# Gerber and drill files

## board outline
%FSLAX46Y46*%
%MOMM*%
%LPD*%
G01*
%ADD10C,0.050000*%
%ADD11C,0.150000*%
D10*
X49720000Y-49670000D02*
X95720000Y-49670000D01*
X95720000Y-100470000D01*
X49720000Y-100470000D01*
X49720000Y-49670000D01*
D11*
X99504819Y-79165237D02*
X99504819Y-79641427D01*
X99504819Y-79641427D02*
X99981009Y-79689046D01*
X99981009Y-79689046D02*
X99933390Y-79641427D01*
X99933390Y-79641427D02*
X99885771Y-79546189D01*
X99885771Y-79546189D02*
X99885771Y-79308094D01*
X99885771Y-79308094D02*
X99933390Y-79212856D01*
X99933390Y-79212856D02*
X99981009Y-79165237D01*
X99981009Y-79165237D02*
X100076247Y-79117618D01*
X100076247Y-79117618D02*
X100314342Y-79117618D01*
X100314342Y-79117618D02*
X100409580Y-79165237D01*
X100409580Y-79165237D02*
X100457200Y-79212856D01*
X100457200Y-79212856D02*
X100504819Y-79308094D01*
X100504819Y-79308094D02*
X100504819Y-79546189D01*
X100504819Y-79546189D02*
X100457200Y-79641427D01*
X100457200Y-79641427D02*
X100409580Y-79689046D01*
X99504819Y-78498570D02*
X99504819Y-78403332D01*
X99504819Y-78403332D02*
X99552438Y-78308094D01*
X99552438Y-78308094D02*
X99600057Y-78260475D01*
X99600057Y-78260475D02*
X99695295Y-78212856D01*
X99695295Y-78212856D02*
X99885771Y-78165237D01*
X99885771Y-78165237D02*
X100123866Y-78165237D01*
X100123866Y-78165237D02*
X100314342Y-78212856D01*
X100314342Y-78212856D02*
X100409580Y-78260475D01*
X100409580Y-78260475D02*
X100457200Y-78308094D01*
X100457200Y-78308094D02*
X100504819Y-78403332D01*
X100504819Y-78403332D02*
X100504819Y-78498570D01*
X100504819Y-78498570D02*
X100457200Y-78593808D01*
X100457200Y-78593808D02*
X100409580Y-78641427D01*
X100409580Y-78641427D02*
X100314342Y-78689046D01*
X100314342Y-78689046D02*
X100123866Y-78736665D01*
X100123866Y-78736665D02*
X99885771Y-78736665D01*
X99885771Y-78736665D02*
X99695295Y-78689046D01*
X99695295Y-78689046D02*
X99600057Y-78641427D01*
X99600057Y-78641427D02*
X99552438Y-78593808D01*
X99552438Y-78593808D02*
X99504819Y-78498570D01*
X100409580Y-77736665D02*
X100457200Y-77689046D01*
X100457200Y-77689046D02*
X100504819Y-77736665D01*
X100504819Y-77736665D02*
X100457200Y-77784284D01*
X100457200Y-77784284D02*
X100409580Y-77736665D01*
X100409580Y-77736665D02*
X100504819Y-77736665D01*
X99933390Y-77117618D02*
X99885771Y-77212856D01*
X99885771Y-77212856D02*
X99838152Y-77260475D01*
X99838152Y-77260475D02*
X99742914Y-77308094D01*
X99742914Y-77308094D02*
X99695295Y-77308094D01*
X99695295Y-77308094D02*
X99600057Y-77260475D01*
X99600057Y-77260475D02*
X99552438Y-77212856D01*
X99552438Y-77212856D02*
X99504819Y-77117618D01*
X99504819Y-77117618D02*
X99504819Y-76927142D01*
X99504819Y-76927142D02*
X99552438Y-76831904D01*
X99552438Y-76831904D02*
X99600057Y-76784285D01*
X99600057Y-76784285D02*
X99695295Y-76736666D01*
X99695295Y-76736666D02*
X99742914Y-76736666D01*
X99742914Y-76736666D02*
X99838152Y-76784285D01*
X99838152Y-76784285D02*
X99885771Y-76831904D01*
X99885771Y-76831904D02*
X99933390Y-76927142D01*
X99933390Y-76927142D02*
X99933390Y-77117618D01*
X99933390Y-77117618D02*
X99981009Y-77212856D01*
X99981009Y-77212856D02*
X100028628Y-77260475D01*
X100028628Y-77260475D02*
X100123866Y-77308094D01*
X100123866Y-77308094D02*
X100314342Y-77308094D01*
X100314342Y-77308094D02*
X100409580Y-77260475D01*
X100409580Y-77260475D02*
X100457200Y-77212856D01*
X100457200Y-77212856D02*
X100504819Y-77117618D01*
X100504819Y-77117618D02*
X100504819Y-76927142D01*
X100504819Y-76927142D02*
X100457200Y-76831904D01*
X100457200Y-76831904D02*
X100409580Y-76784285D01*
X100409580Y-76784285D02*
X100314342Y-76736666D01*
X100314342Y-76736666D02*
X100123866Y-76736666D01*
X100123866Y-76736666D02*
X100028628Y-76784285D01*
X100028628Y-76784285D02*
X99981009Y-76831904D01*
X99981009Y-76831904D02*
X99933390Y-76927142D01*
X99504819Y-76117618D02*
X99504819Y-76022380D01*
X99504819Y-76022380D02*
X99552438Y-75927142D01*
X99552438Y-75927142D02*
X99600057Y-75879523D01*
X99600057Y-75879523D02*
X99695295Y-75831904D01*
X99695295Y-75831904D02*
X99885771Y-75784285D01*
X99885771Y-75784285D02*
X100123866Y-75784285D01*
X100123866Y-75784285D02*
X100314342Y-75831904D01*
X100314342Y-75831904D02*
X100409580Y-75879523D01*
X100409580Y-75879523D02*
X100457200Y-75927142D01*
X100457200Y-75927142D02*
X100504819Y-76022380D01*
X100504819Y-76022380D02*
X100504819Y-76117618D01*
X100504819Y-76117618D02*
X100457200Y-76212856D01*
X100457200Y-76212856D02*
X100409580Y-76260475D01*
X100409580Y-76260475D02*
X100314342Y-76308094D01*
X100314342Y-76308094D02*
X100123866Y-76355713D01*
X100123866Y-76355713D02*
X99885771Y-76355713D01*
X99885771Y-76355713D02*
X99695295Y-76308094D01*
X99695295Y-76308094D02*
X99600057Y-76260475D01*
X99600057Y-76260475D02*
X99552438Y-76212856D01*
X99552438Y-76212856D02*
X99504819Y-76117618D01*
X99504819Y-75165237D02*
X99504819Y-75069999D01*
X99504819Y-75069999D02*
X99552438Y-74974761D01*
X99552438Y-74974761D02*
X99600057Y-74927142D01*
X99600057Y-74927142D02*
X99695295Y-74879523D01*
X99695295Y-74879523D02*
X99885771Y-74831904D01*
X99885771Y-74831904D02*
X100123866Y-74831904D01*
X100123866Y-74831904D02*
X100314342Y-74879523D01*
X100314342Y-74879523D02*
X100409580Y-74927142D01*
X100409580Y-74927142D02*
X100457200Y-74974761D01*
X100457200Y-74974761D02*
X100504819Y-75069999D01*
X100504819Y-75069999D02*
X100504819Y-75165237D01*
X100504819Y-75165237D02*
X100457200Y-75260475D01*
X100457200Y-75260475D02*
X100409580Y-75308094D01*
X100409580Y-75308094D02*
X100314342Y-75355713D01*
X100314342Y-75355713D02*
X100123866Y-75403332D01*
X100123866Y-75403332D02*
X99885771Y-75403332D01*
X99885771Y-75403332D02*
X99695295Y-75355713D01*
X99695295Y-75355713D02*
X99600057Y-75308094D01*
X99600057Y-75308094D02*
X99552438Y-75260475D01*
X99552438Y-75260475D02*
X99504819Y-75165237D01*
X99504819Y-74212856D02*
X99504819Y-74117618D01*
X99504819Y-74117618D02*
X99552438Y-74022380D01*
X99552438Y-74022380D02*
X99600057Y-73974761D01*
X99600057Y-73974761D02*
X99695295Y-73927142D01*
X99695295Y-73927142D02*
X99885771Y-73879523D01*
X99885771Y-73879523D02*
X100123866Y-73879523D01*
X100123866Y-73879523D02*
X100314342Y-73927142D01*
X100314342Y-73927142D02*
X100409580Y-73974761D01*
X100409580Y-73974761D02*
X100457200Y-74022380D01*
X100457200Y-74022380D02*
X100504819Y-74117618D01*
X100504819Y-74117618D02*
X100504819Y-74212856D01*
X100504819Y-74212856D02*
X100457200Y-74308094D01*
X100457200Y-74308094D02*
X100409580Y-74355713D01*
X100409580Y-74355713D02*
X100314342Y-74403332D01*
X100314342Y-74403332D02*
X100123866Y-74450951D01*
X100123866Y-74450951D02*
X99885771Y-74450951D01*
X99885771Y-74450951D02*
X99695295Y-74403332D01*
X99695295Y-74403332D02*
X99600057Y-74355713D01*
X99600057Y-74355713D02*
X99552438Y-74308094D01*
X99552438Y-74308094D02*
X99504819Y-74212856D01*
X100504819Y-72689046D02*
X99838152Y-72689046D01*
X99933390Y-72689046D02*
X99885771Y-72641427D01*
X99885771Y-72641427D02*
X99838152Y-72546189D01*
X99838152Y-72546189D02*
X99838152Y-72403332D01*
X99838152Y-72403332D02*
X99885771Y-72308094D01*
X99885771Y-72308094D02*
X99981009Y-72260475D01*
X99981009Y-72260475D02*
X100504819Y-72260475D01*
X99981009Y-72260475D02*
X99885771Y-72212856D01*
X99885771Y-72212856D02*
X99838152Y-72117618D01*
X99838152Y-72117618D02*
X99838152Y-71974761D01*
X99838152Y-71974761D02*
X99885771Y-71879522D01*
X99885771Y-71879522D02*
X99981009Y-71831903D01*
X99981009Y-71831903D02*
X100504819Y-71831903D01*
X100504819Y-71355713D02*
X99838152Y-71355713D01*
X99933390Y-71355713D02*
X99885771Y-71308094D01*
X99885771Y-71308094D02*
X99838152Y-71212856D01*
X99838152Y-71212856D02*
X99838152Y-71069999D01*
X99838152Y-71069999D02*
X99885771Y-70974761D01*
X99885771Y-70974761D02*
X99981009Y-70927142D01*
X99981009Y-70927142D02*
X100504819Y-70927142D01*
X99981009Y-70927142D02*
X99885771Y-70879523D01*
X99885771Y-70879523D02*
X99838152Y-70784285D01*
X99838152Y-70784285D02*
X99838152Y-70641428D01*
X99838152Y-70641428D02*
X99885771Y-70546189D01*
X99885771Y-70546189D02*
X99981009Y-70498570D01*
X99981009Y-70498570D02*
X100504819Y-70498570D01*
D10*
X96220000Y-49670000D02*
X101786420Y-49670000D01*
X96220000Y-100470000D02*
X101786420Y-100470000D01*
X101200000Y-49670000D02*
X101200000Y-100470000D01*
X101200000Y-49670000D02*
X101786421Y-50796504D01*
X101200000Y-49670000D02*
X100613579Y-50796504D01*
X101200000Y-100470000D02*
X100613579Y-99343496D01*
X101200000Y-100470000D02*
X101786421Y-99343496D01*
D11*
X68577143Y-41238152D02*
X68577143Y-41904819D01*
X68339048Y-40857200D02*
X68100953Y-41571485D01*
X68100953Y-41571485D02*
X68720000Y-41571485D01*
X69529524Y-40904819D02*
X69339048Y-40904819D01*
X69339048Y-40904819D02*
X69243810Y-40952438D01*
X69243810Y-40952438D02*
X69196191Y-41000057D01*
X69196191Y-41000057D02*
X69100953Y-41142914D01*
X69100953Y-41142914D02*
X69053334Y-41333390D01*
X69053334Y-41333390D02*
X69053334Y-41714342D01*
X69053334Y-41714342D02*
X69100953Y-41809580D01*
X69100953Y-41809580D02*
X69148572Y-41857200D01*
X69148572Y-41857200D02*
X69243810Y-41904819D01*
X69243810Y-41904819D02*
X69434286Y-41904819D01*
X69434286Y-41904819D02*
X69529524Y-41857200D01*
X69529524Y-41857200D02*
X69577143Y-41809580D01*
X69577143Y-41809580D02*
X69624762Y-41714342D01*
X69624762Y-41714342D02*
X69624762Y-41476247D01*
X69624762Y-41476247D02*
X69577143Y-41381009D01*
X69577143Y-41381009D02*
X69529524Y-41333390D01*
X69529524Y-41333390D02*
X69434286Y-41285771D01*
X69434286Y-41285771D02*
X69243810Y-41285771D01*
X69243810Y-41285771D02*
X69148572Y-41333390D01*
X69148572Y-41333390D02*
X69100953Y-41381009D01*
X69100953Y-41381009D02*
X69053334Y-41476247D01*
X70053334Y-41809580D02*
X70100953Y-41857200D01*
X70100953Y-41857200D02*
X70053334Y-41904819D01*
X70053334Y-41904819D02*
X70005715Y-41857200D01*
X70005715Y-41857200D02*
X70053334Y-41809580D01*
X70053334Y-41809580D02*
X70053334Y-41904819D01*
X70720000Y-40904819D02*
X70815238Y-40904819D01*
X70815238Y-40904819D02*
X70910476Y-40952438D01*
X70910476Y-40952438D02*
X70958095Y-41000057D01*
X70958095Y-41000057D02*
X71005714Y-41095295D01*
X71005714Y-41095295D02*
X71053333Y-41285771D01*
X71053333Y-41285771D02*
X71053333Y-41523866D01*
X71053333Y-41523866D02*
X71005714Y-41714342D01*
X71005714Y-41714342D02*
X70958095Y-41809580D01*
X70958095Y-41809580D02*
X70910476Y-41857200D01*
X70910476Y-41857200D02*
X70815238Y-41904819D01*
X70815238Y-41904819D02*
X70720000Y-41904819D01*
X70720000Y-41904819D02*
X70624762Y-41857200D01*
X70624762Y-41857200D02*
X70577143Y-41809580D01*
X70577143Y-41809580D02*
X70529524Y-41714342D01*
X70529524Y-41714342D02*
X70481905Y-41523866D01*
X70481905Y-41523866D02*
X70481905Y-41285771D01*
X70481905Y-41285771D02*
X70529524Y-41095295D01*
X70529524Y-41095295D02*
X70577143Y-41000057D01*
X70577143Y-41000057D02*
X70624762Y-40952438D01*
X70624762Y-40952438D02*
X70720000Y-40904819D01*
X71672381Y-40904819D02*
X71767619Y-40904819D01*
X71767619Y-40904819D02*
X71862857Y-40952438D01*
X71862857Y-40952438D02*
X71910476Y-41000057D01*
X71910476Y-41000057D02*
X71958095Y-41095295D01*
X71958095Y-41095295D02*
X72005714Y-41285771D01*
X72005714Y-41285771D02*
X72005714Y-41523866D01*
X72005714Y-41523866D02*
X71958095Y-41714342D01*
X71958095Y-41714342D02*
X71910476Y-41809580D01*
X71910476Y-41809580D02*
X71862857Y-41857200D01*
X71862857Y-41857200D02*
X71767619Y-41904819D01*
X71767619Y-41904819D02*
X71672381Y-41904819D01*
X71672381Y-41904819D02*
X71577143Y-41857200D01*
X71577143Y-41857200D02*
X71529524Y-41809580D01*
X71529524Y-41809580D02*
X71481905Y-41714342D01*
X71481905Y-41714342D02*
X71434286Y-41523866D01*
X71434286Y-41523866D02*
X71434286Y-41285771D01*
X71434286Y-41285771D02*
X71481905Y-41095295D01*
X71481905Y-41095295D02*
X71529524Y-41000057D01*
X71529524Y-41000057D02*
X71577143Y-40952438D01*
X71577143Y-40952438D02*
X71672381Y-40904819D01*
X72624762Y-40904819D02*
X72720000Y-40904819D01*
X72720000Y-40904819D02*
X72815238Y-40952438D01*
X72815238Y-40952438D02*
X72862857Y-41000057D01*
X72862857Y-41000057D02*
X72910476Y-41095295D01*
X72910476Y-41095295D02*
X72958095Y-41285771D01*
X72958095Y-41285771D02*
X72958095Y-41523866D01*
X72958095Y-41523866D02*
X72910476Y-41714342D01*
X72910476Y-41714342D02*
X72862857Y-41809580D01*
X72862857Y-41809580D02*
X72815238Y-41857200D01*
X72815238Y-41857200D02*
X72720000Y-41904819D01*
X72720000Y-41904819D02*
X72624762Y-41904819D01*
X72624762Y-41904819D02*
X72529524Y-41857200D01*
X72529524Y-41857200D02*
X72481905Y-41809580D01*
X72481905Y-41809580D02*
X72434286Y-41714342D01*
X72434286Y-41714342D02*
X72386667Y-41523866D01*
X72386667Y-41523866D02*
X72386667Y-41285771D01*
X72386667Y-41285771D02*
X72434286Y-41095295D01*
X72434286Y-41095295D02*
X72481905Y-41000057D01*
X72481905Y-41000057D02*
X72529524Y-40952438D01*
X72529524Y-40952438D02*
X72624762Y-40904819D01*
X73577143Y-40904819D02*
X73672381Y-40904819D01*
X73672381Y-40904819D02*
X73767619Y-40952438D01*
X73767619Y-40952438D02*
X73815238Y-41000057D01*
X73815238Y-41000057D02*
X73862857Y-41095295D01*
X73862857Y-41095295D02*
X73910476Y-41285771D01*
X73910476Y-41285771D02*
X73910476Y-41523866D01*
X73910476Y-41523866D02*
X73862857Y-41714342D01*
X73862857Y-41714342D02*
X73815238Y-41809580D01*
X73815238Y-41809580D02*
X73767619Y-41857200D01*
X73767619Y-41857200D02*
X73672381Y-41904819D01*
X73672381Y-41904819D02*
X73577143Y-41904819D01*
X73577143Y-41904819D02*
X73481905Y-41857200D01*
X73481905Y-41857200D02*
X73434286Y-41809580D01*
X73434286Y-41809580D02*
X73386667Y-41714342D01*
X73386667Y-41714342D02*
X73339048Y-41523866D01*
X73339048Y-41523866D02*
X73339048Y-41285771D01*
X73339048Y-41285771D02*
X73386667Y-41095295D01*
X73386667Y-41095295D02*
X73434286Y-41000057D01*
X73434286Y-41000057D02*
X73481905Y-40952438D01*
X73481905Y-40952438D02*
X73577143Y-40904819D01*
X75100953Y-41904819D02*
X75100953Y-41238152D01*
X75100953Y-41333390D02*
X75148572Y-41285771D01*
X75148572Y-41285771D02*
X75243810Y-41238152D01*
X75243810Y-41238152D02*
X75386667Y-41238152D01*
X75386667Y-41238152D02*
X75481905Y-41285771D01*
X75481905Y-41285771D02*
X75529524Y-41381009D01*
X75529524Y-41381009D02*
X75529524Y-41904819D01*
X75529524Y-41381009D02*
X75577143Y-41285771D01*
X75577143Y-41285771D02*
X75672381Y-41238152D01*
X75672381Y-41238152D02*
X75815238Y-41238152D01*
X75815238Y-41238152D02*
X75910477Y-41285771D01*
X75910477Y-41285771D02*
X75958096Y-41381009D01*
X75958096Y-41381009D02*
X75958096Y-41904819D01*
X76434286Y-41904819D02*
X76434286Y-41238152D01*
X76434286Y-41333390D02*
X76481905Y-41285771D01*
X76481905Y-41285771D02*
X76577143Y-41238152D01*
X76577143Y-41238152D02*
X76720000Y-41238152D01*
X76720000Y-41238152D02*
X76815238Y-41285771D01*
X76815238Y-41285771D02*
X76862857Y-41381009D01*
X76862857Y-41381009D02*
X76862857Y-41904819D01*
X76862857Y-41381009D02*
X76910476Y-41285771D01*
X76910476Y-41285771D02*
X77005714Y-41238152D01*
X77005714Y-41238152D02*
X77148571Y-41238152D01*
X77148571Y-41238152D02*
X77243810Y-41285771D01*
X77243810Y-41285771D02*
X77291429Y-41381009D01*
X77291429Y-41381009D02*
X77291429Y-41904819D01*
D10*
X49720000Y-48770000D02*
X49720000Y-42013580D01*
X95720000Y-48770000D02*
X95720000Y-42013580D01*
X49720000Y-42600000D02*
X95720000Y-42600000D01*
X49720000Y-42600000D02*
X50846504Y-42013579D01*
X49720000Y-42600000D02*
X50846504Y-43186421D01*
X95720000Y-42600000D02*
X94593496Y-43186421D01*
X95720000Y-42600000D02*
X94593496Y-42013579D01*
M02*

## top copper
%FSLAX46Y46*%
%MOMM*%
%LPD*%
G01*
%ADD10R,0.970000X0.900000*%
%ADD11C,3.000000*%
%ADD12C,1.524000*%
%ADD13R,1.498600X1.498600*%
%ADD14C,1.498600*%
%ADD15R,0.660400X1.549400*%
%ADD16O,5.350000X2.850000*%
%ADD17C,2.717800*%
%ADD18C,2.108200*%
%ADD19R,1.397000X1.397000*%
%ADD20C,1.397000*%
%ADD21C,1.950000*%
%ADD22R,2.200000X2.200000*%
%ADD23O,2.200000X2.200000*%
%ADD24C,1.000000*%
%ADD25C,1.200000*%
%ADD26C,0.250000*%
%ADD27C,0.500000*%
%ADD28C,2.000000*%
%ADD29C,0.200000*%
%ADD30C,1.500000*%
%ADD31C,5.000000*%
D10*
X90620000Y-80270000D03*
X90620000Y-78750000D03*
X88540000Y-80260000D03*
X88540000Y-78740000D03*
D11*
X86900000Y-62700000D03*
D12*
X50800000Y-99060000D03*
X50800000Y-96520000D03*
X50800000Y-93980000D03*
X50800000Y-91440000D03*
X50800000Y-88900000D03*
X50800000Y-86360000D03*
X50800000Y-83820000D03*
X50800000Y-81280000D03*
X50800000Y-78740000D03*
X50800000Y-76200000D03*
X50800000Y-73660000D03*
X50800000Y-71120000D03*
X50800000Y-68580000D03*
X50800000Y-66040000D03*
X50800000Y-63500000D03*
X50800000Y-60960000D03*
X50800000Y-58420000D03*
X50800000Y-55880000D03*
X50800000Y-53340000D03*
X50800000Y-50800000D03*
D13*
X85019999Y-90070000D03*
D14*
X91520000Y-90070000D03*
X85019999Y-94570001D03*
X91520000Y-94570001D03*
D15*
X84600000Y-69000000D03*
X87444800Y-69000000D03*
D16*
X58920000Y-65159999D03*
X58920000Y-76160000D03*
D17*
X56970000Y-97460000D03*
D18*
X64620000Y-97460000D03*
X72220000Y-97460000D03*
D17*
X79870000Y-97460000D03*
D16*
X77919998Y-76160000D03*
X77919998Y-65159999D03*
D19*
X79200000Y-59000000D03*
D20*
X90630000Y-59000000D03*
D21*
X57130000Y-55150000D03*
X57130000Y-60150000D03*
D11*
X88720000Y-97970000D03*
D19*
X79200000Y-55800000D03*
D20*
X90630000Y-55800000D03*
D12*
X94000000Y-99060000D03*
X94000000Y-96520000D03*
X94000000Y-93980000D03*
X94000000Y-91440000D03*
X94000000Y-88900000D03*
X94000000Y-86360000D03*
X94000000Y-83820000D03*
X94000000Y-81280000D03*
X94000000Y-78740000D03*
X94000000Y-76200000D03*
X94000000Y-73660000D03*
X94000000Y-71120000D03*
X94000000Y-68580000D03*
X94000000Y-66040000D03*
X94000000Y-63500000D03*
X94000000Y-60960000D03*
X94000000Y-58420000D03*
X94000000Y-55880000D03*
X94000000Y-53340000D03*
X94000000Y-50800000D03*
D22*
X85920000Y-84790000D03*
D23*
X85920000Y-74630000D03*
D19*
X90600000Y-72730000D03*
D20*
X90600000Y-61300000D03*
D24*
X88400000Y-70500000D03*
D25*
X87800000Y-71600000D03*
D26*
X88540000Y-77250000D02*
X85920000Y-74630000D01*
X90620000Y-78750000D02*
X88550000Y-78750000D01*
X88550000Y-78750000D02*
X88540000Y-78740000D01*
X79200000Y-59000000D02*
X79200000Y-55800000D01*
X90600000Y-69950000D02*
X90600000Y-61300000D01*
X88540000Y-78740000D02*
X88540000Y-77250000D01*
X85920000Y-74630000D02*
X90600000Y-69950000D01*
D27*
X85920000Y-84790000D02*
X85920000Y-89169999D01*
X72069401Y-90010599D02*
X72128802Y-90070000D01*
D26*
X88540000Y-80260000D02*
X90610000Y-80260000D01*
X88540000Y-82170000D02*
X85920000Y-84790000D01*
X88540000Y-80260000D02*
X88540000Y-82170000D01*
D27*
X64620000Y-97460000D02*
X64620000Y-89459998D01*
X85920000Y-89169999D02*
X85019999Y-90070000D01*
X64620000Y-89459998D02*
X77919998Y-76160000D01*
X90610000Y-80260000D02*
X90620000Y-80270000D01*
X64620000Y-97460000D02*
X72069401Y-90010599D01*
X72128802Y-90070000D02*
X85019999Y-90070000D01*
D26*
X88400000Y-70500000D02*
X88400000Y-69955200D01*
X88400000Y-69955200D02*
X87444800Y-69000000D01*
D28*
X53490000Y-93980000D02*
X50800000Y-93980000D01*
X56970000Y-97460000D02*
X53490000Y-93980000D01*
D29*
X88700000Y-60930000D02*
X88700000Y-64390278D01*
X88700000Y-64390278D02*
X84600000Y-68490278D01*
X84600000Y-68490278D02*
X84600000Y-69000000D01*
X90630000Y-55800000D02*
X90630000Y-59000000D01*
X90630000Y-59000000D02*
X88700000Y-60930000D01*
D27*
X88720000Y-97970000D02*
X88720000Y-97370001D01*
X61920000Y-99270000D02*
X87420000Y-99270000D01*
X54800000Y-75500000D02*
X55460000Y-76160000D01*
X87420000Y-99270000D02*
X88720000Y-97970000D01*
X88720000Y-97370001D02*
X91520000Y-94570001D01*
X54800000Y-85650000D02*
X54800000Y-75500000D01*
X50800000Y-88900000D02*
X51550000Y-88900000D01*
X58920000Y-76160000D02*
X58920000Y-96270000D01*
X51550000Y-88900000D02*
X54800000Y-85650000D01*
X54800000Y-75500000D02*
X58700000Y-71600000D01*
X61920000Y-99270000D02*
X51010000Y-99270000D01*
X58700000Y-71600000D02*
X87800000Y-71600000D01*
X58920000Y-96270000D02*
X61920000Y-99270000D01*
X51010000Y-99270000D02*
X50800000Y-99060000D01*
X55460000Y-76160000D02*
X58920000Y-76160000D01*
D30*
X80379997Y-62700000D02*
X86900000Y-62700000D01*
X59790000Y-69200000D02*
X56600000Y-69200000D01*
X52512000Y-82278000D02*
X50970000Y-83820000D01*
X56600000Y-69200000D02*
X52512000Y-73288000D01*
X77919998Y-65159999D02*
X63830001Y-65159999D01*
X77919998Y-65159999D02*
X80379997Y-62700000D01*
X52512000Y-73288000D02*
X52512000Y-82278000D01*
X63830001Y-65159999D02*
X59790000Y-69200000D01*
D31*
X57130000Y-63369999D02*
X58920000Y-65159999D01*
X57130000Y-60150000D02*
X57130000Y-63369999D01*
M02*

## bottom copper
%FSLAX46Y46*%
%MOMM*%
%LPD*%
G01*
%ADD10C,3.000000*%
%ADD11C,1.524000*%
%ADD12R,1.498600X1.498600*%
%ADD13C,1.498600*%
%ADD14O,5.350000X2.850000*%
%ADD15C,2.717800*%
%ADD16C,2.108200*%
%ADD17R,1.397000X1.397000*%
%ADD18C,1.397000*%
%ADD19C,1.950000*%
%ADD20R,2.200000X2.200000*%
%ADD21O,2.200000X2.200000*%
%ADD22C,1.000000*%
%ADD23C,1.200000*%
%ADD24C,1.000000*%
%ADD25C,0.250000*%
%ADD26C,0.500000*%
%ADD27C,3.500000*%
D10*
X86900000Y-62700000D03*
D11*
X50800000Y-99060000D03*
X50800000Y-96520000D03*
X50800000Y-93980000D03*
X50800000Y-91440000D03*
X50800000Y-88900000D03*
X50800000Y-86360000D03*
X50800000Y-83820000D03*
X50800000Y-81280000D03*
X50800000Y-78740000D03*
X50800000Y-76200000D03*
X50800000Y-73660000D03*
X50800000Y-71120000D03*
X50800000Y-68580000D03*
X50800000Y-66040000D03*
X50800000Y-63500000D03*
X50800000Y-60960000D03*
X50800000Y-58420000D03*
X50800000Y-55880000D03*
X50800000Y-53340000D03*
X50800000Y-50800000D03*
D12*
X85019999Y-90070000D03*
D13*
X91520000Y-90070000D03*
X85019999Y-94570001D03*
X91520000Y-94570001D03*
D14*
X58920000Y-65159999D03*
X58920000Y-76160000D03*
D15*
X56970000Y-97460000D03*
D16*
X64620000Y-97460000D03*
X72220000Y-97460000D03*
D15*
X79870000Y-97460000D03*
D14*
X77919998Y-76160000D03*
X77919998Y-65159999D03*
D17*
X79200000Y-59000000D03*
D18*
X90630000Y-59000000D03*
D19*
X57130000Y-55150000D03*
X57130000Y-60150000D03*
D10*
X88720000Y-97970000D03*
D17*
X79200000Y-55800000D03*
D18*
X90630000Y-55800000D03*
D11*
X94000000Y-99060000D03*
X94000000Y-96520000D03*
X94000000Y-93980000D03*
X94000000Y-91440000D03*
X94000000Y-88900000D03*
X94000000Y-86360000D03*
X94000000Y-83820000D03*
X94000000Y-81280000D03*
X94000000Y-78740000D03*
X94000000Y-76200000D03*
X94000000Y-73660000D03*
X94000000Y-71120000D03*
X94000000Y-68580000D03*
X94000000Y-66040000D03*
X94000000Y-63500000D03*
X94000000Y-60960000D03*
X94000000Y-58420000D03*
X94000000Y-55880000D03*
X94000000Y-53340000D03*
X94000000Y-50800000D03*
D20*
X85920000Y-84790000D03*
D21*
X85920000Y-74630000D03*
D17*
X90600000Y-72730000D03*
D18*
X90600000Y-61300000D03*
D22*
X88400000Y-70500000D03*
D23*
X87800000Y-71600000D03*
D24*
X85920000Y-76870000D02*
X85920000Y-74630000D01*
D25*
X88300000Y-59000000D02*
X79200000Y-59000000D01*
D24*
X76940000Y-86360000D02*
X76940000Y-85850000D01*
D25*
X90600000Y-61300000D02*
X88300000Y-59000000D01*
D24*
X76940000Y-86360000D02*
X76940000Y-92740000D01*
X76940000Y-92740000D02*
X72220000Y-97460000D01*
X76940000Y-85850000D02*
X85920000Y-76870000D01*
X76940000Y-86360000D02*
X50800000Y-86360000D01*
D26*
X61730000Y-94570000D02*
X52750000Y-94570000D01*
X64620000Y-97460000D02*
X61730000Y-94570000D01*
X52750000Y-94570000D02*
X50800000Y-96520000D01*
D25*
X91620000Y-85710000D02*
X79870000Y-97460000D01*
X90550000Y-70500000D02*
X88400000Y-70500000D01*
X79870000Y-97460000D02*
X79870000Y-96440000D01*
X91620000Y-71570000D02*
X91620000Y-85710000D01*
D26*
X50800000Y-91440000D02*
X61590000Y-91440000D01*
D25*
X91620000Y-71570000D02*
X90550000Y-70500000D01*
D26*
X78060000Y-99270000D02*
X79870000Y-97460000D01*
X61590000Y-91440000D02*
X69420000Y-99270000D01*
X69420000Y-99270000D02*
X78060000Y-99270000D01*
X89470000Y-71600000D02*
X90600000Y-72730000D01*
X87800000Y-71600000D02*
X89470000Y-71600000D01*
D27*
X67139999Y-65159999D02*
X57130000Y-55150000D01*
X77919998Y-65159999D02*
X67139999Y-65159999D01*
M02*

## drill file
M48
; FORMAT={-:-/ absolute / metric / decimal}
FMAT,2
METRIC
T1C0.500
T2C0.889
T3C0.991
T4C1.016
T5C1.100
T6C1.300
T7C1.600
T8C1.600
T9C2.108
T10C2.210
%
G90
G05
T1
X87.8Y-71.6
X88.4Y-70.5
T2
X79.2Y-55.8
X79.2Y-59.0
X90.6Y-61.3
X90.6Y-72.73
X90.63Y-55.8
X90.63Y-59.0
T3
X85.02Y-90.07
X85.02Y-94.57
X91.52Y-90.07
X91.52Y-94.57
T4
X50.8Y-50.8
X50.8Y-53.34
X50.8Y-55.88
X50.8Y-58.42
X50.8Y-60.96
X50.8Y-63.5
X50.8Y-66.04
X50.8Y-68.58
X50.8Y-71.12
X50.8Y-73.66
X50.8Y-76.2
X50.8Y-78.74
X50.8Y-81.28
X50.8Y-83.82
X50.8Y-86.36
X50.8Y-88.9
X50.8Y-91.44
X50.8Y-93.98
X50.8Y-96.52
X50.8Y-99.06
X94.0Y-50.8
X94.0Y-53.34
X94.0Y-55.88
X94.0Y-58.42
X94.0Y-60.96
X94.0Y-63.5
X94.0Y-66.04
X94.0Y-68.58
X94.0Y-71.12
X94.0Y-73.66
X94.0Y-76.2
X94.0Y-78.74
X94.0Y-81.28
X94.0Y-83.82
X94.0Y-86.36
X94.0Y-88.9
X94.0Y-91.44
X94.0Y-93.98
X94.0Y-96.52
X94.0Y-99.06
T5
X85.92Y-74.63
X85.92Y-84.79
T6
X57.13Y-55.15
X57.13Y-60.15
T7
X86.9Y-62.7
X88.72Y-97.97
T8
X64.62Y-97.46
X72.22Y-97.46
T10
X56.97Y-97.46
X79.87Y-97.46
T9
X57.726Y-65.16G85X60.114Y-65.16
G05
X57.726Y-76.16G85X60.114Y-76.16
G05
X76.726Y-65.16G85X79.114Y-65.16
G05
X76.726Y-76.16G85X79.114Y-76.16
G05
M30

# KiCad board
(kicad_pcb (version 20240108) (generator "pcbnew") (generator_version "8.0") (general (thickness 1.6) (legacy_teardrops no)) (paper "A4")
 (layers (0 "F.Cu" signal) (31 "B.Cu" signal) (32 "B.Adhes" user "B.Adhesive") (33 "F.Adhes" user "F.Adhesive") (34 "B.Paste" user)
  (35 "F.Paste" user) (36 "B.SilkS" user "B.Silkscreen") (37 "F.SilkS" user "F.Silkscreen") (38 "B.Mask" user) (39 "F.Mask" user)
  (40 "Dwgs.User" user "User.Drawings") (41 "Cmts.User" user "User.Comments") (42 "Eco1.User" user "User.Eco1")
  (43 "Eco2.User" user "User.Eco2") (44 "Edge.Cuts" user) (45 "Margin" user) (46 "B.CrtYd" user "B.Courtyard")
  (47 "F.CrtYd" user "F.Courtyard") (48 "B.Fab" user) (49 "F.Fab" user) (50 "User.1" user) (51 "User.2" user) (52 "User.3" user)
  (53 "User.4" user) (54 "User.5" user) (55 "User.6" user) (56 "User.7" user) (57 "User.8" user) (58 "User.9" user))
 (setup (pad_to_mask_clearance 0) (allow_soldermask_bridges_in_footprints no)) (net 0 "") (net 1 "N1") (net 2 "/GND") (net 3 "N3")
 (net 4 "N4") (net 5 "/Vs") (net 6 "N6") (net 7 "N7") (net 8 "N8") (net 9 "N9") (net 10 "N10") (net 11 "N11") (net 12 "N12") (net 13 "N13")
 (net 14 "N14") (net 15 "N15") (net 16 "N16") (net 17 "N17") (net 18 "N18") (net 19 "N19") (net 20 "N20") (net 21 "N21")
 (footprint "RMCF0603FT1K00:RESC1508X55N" (layer "F.Cu") (at 90.62 79.51 90)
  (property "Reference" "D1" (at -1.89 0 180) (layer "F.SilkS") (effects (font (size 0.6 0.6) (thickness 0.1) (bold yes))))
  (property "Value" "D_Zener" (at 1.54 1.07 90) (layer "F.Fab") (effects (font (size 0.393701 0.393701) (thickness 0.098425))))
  (pad "1" smd rect (at -0.76 0 90) (size 0.9 0.97) (layers "F.Cu" "F.Paste" "F.Mask") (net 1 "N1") (solder_mask_margin 0.102))
  (pad "2" smd rect (at 0.76 0 90) (size 0.9 0.97) (layers "F.Cu" "F.Paste" "F.Mask") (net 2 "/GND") (solder_mask_margin 0.102)))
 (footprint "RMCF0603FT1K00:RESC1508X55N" (layer "F.Cu") (at 88.54 79.5 90)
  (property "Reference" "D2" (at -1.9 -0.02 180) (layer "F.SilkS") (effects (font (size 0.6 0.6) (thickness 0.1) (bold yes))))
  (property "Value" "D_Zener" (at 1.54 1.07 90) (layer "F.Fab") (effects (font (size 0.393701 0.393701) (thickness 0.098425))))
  (pad "1" smd rect (at -0.76 0 90) (size 0.9 0.97) (layers "F.Cu" "F.Paste" "F.Mask") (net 1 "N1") (solder_mask_margin 0.102))
  (pad "2" smd rect (at 0.76 0 90) (size 0.9 0.97) (layers "F.Cu" "F.Paste" "F.Mask") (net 2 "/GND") (solder_mask_margin 0.102)))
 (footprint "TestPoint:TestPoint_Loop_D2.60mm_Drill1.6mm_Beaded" (layer "F.Cu") (at 86.9 62.7)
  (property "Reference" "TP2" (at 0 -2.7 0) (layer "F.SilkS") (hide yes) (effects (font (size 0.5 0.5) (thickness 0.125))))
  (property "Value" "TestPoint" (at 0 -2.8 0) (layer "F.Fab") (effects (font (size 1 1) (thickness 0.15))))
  (pad "1" thru_hole circle (at 0 0) (size 3 3) (drill 1.6) (layers "*.Cu" "*.Mask") (remove_unused_layers no) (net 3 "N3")))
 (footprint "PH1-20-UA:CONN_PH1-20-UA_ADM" (layer "F.Cu") (at 50.8 99.06 90)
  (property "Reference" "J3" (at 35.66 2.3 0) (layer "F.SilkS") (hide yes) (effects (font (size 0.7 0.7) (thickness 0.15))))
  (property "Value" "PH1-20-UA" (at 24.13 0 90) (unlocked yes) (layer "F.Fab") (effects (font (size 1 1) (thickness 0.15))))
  (pad "1" thru_hole circle (at 0 0 90) (size 1.524 1.524) (drill 1.016) (layers "*.Cu" "*.Mask") (remove_unused_layers no) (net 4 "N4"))
  (pad "2" thru_hole circle (at 2.54 0 90) (size 1.524 1.524) (drill 1.016) (layers "*.Cu" "*.Mask") (remove_unused_layers no) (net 1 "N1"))
  (pad "3" thru_hole circle (at 5.08 0 90) (size 1.524 1.524) (drill 1.016) (layers "*.Cu" "*.Mask") (remove_unused_layers no) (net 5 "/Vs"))
  (pad "4" thru_hole circle (at 7.62 0 90) (size 1.524 1.524) (drill 1.016) (layers "*.Cu" "*.Mask") (remove_unused_layers no) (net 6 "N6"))
  (pad "5" thru_hole circle (at 10.16 0 90) (size 1.524 1.524) (drill 1.016) (layers "*.Cu" "*.Mask") (remove_unused_layers no) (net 4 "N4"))
  (pad "6" thru_hole circle (at 12.7 0 90) (size 1.524 1.524) (drill 1.016) (layers "*.Cu" "*.Mask") (remove_unused_layers no)
   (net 2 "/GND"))
  (pad "7" thru_hole circle (at 15.24 0 90) (size 1.524 1.524) (drill 1.016) (layers "*.Cu" "*.Mask") (remove_unused_layers no) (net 3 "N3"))
  (pad "8" thru_hole circle (at 17.78 0 90) (size 1.524 1.524) (drill 1.016) (layers "*.Cu" "*.Mask") (remove_unused_layers no) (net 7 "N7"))
  (pad "9" thru_hole circle (at 20.32 0 90) (size 1.524 1.524) (drill 1.016) (layers "*.Cu" "*.Mask") (remove_unused_layers no) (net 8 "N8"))
  (pad "10" thru_hole circle (at 22.86 0 90) (size 1.524 1.524) (drill 1.016) (layers "*.Cu" "*.Mask") (remove_unused_layers no)
   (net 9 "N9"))
  (pad "11" thru_hole circle (at 25.4 0 90) (size 1.524 1.524) (drill 1.016) (layers "*.Cu" "*.Mask") (remove_unused_layers no)
   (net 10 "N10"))
  (pad "12" thru_hole circle (at 27.94 0 90) (size 1.524 1.524) (drill 1.016) (layers "*.Cu" "*.Mask") (remove_unused_layers no)
   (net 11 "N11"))
  (pad "13" thru_hole circle (at 30.48 0 90) (size 1.524 1.524) (drill 1.016) (layers "*.Cu" "*.Mask") (remove_unused_layers no)
   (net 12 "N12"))
  (pad "14" thru_hole circle (at 33.02 0 90) (size 1.524 1.524) (drill 1.016) (layers "*.Cu" "*.Mask") (remove_unused_layers no)
   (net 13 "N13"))
  (pad "15" thru_hole circle (at 35.56 0 90) (size 1.524 1.524) (drill 1.016) (layers "*.Cu" "*.Mask") (remove_unused_layers no)
   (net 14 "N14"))
  (pad "16" thru_hole circle (at 38.1 0 90) (size 1.524 1.524) (drill 1.016) (layers "*.Cu" "*.Mask") (remove_unused_layers no)
   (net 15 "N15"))
  (pad "17" thru_hole circle (at 40.64 0 90) (size 1.524 1.524) (drill 1.016) (layers "*.Cu" "*.Mask") (remove_unused_layers no)
   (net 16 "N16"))
  (pad "18" thru_hole circle (at 43.18 0 90) (size 1.524 1.524) (drill 1.016) (layers "*.Cu" "*.Mask") (remove_unused_layers no)
   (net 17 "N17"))
  (pad "19" thru_hole circle (at 45.72 0 90) (size 1.524 1.524) (drill 1.016) (layers "*.Cu" "*.Mask") (remove_unused_layers no)
   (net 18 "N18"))
  (pad "20" thru_hole circle (at 48.26 0 90) (size 1.524 1.524) (drill 1.016) (layers "*.Cu" "*.Mask") (remove_unused_layers no)
   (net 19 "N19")))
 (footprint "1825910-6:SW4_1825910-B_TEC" (layer "F.Cu") (at 91.52 94.570001)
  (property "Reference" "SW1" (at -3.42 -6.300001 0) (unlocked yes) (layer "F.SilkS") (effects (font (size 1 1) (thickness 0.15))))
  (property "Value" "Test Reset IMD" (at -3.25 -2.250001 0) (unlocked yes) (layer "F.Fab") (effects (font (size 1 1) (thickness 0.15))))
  (pad "1" thru_hole rect (at -6.500001 -4.500001) (size 1.4986 1.4986) (drill 0.9906) (layers "*.Cu" "*.Mask") (remove_unused_layers no)
   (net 1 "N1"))
  (pad "2" thru_hole circle (at 0 -4.500001) (size 1.4986 1.4986) (drill 0.9906) (layers "*.Cu" "*.Mask") (remove_unused_layers no)
   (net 4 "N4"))
  (pad "3" thru_hole circle (at -6.500001 0) (size 1.4986 1.4986) (drill 0.9906) (layers "*.Cu" "*.Mask") (remove_unused_layers no))
  (pad "4" thru_hole circle (at 0 0) (size 1.4986 1.4986) (drill 0.9906) (layers "*.Cu" "*.Mask") (remove_unused_layers no)))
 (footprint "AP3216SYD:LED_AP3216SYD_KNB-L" (layer "F.Cu") (at 86.0224 69)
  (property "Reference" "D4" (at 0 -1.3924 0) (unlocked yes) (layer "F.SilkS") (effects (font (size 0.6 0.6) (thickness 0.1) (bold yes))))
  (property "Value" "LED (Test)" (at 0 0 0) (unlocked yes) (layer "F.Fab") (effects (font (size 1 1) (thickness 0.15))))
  (pad "1" smd rect (at -1.4224 0) (size 0.6604 1.5494) (layers "F.Cu" "F.Paste" "F.Mask") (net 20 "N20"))
  (pad "2" smd rect (at 1.4224 0) (size 0.6604 1.5494) (layers "F.Cu" "F.Paste" "F.Mask") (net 6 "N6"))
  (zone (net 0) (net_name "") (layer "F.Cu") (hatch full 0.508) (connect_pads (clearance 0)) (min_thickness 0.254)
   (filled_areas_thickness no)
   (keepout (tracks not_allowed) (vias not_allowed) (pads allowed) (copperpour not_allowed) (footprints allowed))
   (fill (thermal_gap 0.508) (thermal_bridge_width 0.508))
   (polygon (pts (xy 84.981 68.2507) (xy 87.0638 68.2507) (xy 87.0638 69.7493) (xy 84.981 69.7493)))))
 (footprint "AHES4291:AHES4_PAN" (layer "F.Cu") (at 58.919999 65.159998)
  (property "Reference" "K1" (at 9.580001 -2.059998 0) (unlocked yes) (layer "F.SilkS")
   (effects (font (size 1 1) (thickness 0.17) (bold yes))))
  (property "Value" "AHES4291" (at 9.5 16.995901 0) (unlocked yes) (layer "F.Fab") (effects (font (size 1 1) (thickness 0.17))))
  (pad "1" thru_hole oval (at 0.000001 0.000001) (size 5.35 2.85) (drill oval 4.4958 2.1082) (layers "*.Cu" "*.Mask")
   (remove_unused_layers no) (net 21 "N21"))
  (pad "2" thru_hole oval (at 0.000001 11.000002) (size 5.35 2.85) (drill oval 4.4958 2.1082) (layers "*.Cu" "*.Mask")
   (remove_unused_layers no) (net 4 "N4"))
  (pad "3" thru_hole circle (at -1.949999 32.300002) (size 2.7178 2.7178) (drill 2.2098) (layers "*.Cu" "*.Mask") (remove_unused_layers no)
   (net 5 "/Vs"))
  (pad "4" thru_hole circle (at 5.700001 32.300002) (size 2.1082 2.1082) (drill 1.6002) (layers "*.Cu" "*.Mask") (remove_unused_layers no)
   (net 1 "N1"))
  (pad "5" thru_hole circle (at 13.300001 32.300002) (size 2.1082 2.1082) (drill 1.6002) (layers "*.Cu" "*.Mask") (remove_unused_layers no)
   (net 2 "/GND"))
  (pad "6" thru_hole circle (at 20.950001 32.300002) (size 2.7178 2.7178) (drill 2.2098) (layers "*.Cu" "*.Mask") (remove_unused_layers no)
   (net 6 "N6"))
  (pad "7" thru_hole oval (at 18.999999 11.000002) (size 5.35 2.85) (drill oval 4.4958 2.1082) (layers "*.Cu" "*.Mask")
   (remove_unused_layers no) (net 1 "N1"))
  (pad "8" thru_hole oval (at 18.999999 0.000001) (size 5.35 2.85) (drill oval 4.4958 2.1082) (layers "*.Cu" "*.Mask")
   (remove_unused_layers no) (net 3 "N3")))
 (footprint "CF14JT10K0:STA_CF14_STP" (layer "F.Cu") (at 79.2 59)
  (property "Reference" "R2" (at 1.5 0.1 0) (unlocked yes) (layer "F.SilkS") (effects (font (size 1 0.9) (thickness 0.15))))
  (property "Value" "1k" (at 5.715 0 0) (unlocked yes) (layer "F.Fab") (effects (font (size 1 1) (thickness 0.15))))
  (pad "1" thru_hole rect (at 0 0) (size 1.397 1.397) (drill 0.889) (layers "*.Cu" "*.Mask") (remove_unused_layers no) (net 2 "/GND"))
  (pad "2" thru_hole circle (at 11.43 0) (size 1.397 1.397) (drill 0.889) (layers "*.Cu" "*.Mask") (remove_unused_layers no) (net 20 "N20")))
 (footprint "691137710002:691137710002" (layer "F.Cu") (at 57.13 57.65 -90)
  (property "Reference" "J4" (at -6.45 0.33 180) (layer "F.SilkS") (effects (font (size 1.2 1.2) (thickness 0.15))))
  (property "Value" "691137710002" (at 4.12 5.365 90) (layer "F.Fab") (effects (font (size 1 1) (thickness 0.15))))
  (pad "1" thru_hole circle (at -2.5 0 270) (size 1.95 1.95) (drill 1.3) (layers "*.Cu" "*.Mask") (remove_unused_layers no) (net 3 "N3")
   (solder_mask_margin 0.102))
  (pad "2" thru_hole circle (at 2.5 0 270) (size 1.95 1.95) (drill 1.3) (layers "*.Cu" "*.Mask") (remove_unused_layers no) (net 21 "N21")
   (solder_mask_margin 0.102)))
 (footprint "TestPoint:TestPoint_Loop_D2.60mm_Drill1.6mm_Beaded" (layer "F.Cu") (at 88.72 97.97)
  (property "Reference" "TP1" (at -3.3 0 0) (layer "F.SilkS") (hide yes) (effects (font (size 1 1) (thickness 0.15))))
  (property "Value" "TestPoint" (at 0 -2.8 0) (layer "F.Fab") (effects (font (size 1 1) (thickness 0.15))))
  (pad "1" thru_hole circle (at 0 0) (size 3 3) (drill 1.6) (layers "*.Cu" "*.Mask") (remove_unused_layers no) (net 4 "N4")))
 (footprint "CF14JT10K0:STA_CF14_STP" (layer "F.Cu") (at 79.2 55.8)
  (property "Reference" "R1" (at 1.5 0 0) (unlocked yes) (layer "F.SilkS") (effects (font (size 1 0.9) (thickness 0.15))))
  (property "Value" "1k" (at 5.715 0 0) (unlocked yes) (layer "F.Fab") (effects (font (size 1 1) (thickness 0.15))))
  (pad "1" thru_hole rect (at 0 0) (size 1.397 1.397) (drill 0.889) (layers "*.Cu" "*.Mask") (remove_unused_layers no) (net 2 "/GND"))
  (pad "2" thru_hole circle (at 11.43 0) (size 1.397 1.397) (drill 0.889) (layers "*.Cu" "*.Mask") (remove_unused_layers no) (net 20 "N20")))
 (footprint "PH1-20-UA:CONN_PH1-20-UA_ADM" (layer "F.Cu") (at 94 99.06 90)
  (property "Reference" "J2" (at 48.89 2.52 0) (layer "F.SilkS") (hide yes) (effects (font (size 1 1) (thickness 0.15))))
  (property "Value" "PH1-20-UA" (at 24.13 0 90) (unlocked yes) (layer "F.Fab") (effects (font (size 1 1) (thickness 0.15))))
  (pad "1" thru_hole circle (at 0 0 90) (size 1.524 1.524) (drill 1.016) (layers "*.Cu" "*.Mask") (remove_unused_layers no))
  (pad "2" thru_hole circle (at 2.54 0 90) (size 1.524 1.524) (drill 1.016) (layers "*.Cu" "*.Mask") (remove_unused_layers no))
  (pad "3" thru_hole circle (at 5.08 0 90) (size 1.524 1.524) (drill 1.016) (layers "*.Cu" "*.Mask") (remove_unused_layers no))
  (pad "4" thru_hole circle (at 7.62 0 90) (size 1.524 1.524) (drill 1.016) (layers "*.Cu" "*.Mask") (remove_unused_layers no))
  (pad "5" thru_hole circle (at 10.16 0 90) (size 1.524 1.524) (drill 1.016) (layers "*.Cu" "*.Mask") (remove_unused_layers no))
  (pad "6" thru_hole circle (at 12.7 0 90) (size 1.524 1.524) (drill 1.016) (layers "*.Cu" "*.Mask") (remove_unused_layers no))
  (pad "7" thru_hole circle (at 15.24 0 90) (size 1.524 1.524) (drill 1.016) (layers "*.Cu" "*.Mask") (remove_unused_layers no))
  (pad "8" thru_hole circle (at 17.78 0 90) (size 1.524 1.524) (drill 1.016) (layers "*.Cu" "*.Mask") (remove_unused_layers no))
  (pad "9" thru_hole circle (at 20.32 0 90) (size 1.524 1.524) (drill 1.016) (layers "*.Cu" "*.Mask") (remove_unused_layers no))
  (pad "10" thru_hole circle (at 22.86 0 90) (size 1.524 1.524) (drill 1.016) (layers "*.Cu" "*.Mask") (remove_unused_layers no))
  (pad "11" thru_hole circle (at 25.4 0 90) (size 1.524 1.524) (drill 1.016) (layers "*.Cu" "*.Mask") (remove_unused_layers no))
  (pad "12" thru_hole circle (at 27.94 0 90) (size 1.524 1.524) (drill 1.016) (layers "*.Cu" "*.Mask") (remove_unused_layers no))
  (pad "13" thru_hole circle (at 30.48 0 90) (size 1.524 1.524) (drill 1.016) (layers "*.Cu" "*.Mask") (remove_unused_layers no))
  (pad "14" thru_hole circle (at 33.02 0 90) (size 1.524 1.524) (drill 1.016) (layers "*.Cu" "*.Mask") (remove_unused_layers no))
  (pad "15" thru_hole circle (at 35.56 0 90) (size 1.524 1.524) (drill 1.016) (layers "*.Cu" "*.Mask") (remove_unused_layers no))
  (pad "16" thru_hole circle (at 38.1 0 90) (size 1.524 1.524) (drill 1.016) (layers "*.Cu" "*.Mask") (remove_unused_layers no))
  (pad "17" thru_hole circle (at 40.64 0 90) (size 1.524 1.524) (drill 1.016) (layers "*.Cu" "*.Mask") (remove_unused_layers no))
  (pad "18" thru_hole circle (at 43.18 0 90) (size 1.524 1.524) (drill 1.016) (layers "*.Cu" "*.Mask") (remove_unused_layers no))
  (pad "19" thru_hole circle (at 45.72 0 90) (size 1.524 1.524) (drill 1.016) (layers "*.Cu" "*.Mask") (remove_unused_layers no))
  (pad "20" thru_hole circle (at 48.26 0 90) (size 1.524 1.524) (drill 1.016) (layers "*.Cu" "*.Mask") (remove_unused_layers no)))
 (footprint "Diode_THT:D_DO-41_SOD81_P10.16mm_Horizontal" (layer "F.Cu") (at 85.92 84.79 90)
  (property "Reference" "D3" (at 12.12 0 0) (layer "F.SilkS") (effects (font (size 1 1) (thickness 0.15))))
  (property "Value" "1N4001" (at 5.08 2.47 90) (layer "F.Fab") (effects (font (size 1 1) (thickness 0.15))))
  (pad "1" thru_hole rect (at 0 0 90) (size 2.2 2.2) (drill 1.1) (layers "*.Cu" "*.Mask") (remove_unused_layers no) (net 1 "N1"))
  (pad "2" thru_hole oval (at 10.16 0 90) (size 2.2 2.2) (drill 1.1) (layers "*.Cu" "*.Mask") (remove_unused_layers no) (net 2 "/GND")))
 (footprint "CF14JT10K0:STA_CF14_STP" (layer "F.Cu") (at 90.6 72.73 90)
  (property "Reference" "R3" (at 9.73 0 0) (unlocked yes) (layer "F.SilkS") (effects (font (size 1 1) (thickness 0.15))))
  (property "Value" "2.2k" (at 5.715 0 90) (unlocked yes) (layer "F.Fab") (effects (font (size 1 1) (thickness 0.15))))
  (pad "1" thru_hole rect (at 0 0 90) (size 1.397 1.397) (drill 0.889) (layers "*.Cu" "*.Mask") (remove_unused_layers no) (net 4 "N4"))
  (pad "2" thru_hole circle (at 11.43 0 90) (size 1.397 1.397) (drill 0.889) (layers "*.Cu" "*.Mask") (remove_unused_layers no)
   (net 2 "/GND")))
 (gr_rect (start 49.72 49.67) (end 95.72 100.47) (stroke (width 0.05) (type default)) (fill none) (layer "Edge.Cuts"))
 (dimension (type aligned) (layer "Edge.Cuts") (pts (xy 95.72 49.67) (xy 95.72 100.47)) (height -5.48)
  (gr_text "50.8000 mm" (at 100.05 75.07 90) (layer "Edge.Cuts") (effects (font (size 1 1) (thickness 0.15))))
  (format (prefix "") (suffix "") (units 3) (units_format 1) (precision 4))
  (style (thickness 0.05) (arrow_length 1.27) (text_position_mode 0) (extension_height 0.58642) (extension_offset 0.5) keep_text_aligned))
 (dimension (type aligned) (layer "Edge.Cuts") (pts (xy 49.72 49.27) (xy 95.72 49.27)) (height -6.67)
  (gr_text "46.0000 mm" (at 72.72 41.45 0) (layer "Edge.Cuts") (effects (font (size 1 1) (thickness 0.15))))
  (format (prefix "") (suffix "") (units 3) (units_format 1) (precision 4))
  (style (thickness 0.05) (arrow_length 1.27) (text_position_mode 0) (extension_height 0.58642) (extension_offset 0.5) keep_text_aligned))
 (segment (start 88.54 77.25) (end 85.92 74.63) (width 0.25) (layer "F.Cu") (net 2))
 (segment (start 90.62 78.75) (end 88.55 78.75) (width 0.25) (layer "F.Cu") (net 2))
 (segment (start 88.55 78.75) (end 88.54 78.74) (width 0.25) (layer "F.Cu") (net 2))
 (segment (start 79.2 59) (end 79.2 55.8) (width 0.25) (layer "F.Cu") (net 2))
 (segment (start 90.6 69.95) (end 90.6 61.3) (width 0.25) (layer "F.Cu") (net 2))
 (segment (start 88.54 78.74) (end 88.54 77.25) (width 0.25) (layer "F.Cu") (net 2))
 (segment (start 85.92 74.63) (end 90.6 69.95) (width 0.25) (layer "F.Cu") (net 2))
 (segment (start 85.92 76.87) (end 85.92 74.63) (width 1) (layer "B.Cu") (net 2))
 (segment (start 88.3 59) (end 79.2 59) (width 0.25) (layer "B.Cu") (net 2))
 (segment (start 76.94 86.36) (end 76.94 85.85) (width 1) (layer "B.Cu") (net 2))
 (segment (start 90.6 61.3) (end 88.3 59) (width 0.25) (layer "B.Cu") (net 2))
 (segment (start 76.94 86.36) (end 76.94 92.74) (width 1) (layer "B.Cu") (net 2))
 (segment (start 76.94 92.74) (end 72.22 97.46) (width 1) (layer "B.Cu") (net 2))
 (segment (start 76.94 85.85) (end 85.92 76.87) (width 1) (layer "B.Cu") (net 2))
 (segment (start 76.94 86.36) (end 50.8 86.36) (width 1) (layer "B.Cu") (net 2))
 (segment (start 85.92 84.79) (end 85.92 89.169999) (width 0.5) (layer "F.Cu") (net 1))
 (segment (start 72.069401 90.010599) (end 72.128802 90.07) (width 0.5) (layer "F.Cu") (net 1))
 (segment (start 88.54 80.26) (end 90.61 80.26) (width 0.25) (layer "F.Cu") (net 1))
 (segment (start 88.54 82.17) (end 85.92 84.79) (width 0.25) (layer "F.Cu") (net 1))
 (segment (start 88.54 80.26) (end 88.54 82.17) (width 0.25) (layer "F.Cu") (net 1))
 (segment (start 64.62 97.46) (end 64.62 89.459998) (width 0.5) (layer "F.Cu") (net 1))
 (segment (start 85.92 89.169999) (end 85.019999 90.07) (width 0.5) (layer "F.Cu") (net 1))
 (segment (start 64.62 89.459998) (end 77.919998 76.16) (width 0.5) (layer "F.Cu") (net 1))
 (segment (start 90.61 80.26) (end 90.62 80.27) (width 0.5) (layer "F.Cu") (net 1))
 (segment (start 64.62 97.46) (end 72.069401 90.010599) (width 0.5) (layer "F.Cu") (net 1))
 (segment (start 72.128802 90.07) (end 85.019999 90.07) (width 0.5) (layer "F.Cu") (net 1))
 (segment (start 61.73 94.57) (end 52.75 94.57) (width 0.5) (layer "B.Cu") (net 1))
 (segment (start 64.62 97.46) (end 61.73 94.57) (width 0.5) (layer "B.Cu") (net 1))
 (segment (start 52.75 94.57) (end 50.8 96.52) (width 0.5) (layer "B.Cu") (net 1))
 (segment (start 88.4 70.5) (end 88.4 69.9552) (width 0.25) (layer "F.Cu") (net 6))
 (segment (start 88.4 69.9552) (end 87.4448 69) (width 0.25) (layer "F.Cu") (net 6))
 (via (at 88.4 70.5) (size 1) (drill 0.5) (layers "F.Cu" "B.Cu") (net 6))
 (segment (start 91.62 85.71) (end 79.87 97.46) (width 0.25) (layer "B.Cu") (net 6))
 (segment (start 90.55 70.5) (end 88.4 70.5) (width 0.25) (layer "B.Cu") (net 6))
 (segment (start 79.87 97.46) (end 79.87 96.44) (width 0.25) (layer "B.Cu") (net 6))
 (segment (start 91.62 71.57) (end 91.62 85.71) (width 0.25) (layer "B.Cu") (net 6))
 (segment (start 50.8 91.44) (end 61.59 91.44) (width 0.5) (layer "B.Cu") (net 6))
 (segment (start 91.62 71.57) (end 90.55 70.5) (width 0.25) (layer "B.Cu") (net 6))
 (segment (start 78.06 99.27) (end 79.87 97.46) (width 0.5) (layer "B.Cu") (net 6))
 (segment (start 61.59 91.44) (end 69.42 99.27) (width 0.5) (layer "B.Cu") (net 6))
 (segment (start 69.42 99.27) (end 78.06 99.27) (width 0.5) (layer "B.Cu") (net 6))
 (segment (start 53.49 93.98) (end 50.8 93.98) (width 2) (layer "F.Cu") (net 5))
 (segment (start 56.97 97.46) (end 53.49 93.98) (width 2) (layer "F.Cu") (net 5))
 (segment (start 88.7 60.93) (end 88.7 64.390278) (width 0.2) (layer "F.Cu") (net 20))
 (segment (start 88.7 64.390278) (end 84.6 68.490278) (width 0.2) (layer "F.Cu") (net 20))
 (segment (start 84.6 68.490278) (end 84.6 69) (width 0.2) (layer "F.Cu") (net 20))
 (segment (start 90.63 55.8) (end 90.63 59) (width 0.2) (layer "F.Cu") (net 20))
 (segment (start 90.63 59) (end 88.7 60.93) (width 0.2) (layer "F.Cu") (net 20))
 (segment (start 88.72 97.97) (end 88.72 97.370001) (width 0.5) (layer "F.Cu") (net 4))
 (segment (start 61.92 99.27) (end 87.42 99.27) (width 0.5) (layer "F.Cu") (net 4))
 (segment (start 54.8 75.5) (end 55.46 76.16) (width 0.5) (layer "F.Cu") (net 4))
 (segment (start 87.42 99.27) (end 88.72 97.97) (width 0.5) (layer "F.Cu") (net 4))
 (segment (start 88.72 97.370001) (end 91.52 94.570001) (width 0.5) (layer "F.Cu") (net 4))
 (segment (start 54.8 85.65) (end 54.8 75.5) (width 0.5) (layer "F.Cu") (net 4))
 (segment (start 50.8 88.9) (end 51.55 88.9) (width 0.5) (layer "F.Cu") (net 4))
 (segment (start 58.92 76.16) (end 58.92 96.27) (width 0.5) (layer "F.Cu") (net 4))
 (segment (start 51.55 88.9) (end 54.8 85.65) (width 0.5) (layer "F.Cu") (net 4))
 (segment (start 54.8 75.5) (end 58.7 71.6) (width 0.5) (layer "F.Cu") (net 4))
 (segment (start 61.92 99.27) (end 51.01 99.27) (width 0.5) (layer "F.Cu") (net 4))
 (segment (start 58.7 71.6) (end 87.8 71.6) (width 0.5) (layer "F.Cu") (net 4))
 (segment (start 58.92 96.27) (end 61.92 99.27) (width 0.5) (layer "F.Cu") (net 4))
 (segment (start 51.01 99.27) (end 50.8 99.06) (width 0.5) (layer "F.Cu") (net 4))
 (segment (start 55.46 76.16) (end 58.92 76.16) (width 0.5) (layer "F.Cu") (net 4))
 (via (at 87.8 71.6) (size 1.2) (drill 0.5) (layers "F.Cu" "B.Cu") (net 4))
 (segment (start 89.47 71.6) (end 90.6 72.73) (width 0.5) (layer "B.Cu") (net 4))
 (segment (start 87.8 71.6) (end 89.47 71.6) (width 0.5) (layer "B.Cu") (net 4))
 (segment (start 80.379997 62.7) (end 86.9 62.7) (width 1.5) (layer "F.Cu") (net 3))
 (segment (start 59.79 69.2) (end 56.6 69.2) (width 1.5) (layer "F.Cu") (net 3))
 (segment (start 52.512 82.278) (end 50.97 83.82) (width 1.5) (layer "F.Cu") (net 3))
 (segment (start 56.6 69.2) (end 52.512 73.288) (width 1.5) (layer "F.Cu") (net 3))
 (segment (start 77.919998 65.159999) (end 63.830001 65.159999) (width 1.5) (layer "F.Cu") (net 3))
 (segment (start 77.919998 65.159999) (end 80.379997 62.7) (width 1.5) (layer "F.Cu") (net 3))
 (segment (start 52.512 73.288) (end 52.512 82.278) (width 1.5) (layer "F.Cu") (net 3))
 (segment (start 63.830001 65.159999) (end 59.79 69.2) (width 1.5) (layer "F.Cu") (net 3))
 (segment (start 67.139999 65.159999) (end 57.13 55.15) (width 3.5) (layer "B.Cu") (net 3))
 (segment (start 77.919998 65.159999) (end 67.139999 65.159999) (width 3.5) (layer "B.Cu") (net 3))
 (segment (start 57.13 63.369999) (end 58.92 65.159999) (width 5) (layer "F.Cu") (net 21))
 (segment (start 57.13 60.15) (end 57.13 63.369999) (width 5) (layer "F.Cu") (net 21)))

